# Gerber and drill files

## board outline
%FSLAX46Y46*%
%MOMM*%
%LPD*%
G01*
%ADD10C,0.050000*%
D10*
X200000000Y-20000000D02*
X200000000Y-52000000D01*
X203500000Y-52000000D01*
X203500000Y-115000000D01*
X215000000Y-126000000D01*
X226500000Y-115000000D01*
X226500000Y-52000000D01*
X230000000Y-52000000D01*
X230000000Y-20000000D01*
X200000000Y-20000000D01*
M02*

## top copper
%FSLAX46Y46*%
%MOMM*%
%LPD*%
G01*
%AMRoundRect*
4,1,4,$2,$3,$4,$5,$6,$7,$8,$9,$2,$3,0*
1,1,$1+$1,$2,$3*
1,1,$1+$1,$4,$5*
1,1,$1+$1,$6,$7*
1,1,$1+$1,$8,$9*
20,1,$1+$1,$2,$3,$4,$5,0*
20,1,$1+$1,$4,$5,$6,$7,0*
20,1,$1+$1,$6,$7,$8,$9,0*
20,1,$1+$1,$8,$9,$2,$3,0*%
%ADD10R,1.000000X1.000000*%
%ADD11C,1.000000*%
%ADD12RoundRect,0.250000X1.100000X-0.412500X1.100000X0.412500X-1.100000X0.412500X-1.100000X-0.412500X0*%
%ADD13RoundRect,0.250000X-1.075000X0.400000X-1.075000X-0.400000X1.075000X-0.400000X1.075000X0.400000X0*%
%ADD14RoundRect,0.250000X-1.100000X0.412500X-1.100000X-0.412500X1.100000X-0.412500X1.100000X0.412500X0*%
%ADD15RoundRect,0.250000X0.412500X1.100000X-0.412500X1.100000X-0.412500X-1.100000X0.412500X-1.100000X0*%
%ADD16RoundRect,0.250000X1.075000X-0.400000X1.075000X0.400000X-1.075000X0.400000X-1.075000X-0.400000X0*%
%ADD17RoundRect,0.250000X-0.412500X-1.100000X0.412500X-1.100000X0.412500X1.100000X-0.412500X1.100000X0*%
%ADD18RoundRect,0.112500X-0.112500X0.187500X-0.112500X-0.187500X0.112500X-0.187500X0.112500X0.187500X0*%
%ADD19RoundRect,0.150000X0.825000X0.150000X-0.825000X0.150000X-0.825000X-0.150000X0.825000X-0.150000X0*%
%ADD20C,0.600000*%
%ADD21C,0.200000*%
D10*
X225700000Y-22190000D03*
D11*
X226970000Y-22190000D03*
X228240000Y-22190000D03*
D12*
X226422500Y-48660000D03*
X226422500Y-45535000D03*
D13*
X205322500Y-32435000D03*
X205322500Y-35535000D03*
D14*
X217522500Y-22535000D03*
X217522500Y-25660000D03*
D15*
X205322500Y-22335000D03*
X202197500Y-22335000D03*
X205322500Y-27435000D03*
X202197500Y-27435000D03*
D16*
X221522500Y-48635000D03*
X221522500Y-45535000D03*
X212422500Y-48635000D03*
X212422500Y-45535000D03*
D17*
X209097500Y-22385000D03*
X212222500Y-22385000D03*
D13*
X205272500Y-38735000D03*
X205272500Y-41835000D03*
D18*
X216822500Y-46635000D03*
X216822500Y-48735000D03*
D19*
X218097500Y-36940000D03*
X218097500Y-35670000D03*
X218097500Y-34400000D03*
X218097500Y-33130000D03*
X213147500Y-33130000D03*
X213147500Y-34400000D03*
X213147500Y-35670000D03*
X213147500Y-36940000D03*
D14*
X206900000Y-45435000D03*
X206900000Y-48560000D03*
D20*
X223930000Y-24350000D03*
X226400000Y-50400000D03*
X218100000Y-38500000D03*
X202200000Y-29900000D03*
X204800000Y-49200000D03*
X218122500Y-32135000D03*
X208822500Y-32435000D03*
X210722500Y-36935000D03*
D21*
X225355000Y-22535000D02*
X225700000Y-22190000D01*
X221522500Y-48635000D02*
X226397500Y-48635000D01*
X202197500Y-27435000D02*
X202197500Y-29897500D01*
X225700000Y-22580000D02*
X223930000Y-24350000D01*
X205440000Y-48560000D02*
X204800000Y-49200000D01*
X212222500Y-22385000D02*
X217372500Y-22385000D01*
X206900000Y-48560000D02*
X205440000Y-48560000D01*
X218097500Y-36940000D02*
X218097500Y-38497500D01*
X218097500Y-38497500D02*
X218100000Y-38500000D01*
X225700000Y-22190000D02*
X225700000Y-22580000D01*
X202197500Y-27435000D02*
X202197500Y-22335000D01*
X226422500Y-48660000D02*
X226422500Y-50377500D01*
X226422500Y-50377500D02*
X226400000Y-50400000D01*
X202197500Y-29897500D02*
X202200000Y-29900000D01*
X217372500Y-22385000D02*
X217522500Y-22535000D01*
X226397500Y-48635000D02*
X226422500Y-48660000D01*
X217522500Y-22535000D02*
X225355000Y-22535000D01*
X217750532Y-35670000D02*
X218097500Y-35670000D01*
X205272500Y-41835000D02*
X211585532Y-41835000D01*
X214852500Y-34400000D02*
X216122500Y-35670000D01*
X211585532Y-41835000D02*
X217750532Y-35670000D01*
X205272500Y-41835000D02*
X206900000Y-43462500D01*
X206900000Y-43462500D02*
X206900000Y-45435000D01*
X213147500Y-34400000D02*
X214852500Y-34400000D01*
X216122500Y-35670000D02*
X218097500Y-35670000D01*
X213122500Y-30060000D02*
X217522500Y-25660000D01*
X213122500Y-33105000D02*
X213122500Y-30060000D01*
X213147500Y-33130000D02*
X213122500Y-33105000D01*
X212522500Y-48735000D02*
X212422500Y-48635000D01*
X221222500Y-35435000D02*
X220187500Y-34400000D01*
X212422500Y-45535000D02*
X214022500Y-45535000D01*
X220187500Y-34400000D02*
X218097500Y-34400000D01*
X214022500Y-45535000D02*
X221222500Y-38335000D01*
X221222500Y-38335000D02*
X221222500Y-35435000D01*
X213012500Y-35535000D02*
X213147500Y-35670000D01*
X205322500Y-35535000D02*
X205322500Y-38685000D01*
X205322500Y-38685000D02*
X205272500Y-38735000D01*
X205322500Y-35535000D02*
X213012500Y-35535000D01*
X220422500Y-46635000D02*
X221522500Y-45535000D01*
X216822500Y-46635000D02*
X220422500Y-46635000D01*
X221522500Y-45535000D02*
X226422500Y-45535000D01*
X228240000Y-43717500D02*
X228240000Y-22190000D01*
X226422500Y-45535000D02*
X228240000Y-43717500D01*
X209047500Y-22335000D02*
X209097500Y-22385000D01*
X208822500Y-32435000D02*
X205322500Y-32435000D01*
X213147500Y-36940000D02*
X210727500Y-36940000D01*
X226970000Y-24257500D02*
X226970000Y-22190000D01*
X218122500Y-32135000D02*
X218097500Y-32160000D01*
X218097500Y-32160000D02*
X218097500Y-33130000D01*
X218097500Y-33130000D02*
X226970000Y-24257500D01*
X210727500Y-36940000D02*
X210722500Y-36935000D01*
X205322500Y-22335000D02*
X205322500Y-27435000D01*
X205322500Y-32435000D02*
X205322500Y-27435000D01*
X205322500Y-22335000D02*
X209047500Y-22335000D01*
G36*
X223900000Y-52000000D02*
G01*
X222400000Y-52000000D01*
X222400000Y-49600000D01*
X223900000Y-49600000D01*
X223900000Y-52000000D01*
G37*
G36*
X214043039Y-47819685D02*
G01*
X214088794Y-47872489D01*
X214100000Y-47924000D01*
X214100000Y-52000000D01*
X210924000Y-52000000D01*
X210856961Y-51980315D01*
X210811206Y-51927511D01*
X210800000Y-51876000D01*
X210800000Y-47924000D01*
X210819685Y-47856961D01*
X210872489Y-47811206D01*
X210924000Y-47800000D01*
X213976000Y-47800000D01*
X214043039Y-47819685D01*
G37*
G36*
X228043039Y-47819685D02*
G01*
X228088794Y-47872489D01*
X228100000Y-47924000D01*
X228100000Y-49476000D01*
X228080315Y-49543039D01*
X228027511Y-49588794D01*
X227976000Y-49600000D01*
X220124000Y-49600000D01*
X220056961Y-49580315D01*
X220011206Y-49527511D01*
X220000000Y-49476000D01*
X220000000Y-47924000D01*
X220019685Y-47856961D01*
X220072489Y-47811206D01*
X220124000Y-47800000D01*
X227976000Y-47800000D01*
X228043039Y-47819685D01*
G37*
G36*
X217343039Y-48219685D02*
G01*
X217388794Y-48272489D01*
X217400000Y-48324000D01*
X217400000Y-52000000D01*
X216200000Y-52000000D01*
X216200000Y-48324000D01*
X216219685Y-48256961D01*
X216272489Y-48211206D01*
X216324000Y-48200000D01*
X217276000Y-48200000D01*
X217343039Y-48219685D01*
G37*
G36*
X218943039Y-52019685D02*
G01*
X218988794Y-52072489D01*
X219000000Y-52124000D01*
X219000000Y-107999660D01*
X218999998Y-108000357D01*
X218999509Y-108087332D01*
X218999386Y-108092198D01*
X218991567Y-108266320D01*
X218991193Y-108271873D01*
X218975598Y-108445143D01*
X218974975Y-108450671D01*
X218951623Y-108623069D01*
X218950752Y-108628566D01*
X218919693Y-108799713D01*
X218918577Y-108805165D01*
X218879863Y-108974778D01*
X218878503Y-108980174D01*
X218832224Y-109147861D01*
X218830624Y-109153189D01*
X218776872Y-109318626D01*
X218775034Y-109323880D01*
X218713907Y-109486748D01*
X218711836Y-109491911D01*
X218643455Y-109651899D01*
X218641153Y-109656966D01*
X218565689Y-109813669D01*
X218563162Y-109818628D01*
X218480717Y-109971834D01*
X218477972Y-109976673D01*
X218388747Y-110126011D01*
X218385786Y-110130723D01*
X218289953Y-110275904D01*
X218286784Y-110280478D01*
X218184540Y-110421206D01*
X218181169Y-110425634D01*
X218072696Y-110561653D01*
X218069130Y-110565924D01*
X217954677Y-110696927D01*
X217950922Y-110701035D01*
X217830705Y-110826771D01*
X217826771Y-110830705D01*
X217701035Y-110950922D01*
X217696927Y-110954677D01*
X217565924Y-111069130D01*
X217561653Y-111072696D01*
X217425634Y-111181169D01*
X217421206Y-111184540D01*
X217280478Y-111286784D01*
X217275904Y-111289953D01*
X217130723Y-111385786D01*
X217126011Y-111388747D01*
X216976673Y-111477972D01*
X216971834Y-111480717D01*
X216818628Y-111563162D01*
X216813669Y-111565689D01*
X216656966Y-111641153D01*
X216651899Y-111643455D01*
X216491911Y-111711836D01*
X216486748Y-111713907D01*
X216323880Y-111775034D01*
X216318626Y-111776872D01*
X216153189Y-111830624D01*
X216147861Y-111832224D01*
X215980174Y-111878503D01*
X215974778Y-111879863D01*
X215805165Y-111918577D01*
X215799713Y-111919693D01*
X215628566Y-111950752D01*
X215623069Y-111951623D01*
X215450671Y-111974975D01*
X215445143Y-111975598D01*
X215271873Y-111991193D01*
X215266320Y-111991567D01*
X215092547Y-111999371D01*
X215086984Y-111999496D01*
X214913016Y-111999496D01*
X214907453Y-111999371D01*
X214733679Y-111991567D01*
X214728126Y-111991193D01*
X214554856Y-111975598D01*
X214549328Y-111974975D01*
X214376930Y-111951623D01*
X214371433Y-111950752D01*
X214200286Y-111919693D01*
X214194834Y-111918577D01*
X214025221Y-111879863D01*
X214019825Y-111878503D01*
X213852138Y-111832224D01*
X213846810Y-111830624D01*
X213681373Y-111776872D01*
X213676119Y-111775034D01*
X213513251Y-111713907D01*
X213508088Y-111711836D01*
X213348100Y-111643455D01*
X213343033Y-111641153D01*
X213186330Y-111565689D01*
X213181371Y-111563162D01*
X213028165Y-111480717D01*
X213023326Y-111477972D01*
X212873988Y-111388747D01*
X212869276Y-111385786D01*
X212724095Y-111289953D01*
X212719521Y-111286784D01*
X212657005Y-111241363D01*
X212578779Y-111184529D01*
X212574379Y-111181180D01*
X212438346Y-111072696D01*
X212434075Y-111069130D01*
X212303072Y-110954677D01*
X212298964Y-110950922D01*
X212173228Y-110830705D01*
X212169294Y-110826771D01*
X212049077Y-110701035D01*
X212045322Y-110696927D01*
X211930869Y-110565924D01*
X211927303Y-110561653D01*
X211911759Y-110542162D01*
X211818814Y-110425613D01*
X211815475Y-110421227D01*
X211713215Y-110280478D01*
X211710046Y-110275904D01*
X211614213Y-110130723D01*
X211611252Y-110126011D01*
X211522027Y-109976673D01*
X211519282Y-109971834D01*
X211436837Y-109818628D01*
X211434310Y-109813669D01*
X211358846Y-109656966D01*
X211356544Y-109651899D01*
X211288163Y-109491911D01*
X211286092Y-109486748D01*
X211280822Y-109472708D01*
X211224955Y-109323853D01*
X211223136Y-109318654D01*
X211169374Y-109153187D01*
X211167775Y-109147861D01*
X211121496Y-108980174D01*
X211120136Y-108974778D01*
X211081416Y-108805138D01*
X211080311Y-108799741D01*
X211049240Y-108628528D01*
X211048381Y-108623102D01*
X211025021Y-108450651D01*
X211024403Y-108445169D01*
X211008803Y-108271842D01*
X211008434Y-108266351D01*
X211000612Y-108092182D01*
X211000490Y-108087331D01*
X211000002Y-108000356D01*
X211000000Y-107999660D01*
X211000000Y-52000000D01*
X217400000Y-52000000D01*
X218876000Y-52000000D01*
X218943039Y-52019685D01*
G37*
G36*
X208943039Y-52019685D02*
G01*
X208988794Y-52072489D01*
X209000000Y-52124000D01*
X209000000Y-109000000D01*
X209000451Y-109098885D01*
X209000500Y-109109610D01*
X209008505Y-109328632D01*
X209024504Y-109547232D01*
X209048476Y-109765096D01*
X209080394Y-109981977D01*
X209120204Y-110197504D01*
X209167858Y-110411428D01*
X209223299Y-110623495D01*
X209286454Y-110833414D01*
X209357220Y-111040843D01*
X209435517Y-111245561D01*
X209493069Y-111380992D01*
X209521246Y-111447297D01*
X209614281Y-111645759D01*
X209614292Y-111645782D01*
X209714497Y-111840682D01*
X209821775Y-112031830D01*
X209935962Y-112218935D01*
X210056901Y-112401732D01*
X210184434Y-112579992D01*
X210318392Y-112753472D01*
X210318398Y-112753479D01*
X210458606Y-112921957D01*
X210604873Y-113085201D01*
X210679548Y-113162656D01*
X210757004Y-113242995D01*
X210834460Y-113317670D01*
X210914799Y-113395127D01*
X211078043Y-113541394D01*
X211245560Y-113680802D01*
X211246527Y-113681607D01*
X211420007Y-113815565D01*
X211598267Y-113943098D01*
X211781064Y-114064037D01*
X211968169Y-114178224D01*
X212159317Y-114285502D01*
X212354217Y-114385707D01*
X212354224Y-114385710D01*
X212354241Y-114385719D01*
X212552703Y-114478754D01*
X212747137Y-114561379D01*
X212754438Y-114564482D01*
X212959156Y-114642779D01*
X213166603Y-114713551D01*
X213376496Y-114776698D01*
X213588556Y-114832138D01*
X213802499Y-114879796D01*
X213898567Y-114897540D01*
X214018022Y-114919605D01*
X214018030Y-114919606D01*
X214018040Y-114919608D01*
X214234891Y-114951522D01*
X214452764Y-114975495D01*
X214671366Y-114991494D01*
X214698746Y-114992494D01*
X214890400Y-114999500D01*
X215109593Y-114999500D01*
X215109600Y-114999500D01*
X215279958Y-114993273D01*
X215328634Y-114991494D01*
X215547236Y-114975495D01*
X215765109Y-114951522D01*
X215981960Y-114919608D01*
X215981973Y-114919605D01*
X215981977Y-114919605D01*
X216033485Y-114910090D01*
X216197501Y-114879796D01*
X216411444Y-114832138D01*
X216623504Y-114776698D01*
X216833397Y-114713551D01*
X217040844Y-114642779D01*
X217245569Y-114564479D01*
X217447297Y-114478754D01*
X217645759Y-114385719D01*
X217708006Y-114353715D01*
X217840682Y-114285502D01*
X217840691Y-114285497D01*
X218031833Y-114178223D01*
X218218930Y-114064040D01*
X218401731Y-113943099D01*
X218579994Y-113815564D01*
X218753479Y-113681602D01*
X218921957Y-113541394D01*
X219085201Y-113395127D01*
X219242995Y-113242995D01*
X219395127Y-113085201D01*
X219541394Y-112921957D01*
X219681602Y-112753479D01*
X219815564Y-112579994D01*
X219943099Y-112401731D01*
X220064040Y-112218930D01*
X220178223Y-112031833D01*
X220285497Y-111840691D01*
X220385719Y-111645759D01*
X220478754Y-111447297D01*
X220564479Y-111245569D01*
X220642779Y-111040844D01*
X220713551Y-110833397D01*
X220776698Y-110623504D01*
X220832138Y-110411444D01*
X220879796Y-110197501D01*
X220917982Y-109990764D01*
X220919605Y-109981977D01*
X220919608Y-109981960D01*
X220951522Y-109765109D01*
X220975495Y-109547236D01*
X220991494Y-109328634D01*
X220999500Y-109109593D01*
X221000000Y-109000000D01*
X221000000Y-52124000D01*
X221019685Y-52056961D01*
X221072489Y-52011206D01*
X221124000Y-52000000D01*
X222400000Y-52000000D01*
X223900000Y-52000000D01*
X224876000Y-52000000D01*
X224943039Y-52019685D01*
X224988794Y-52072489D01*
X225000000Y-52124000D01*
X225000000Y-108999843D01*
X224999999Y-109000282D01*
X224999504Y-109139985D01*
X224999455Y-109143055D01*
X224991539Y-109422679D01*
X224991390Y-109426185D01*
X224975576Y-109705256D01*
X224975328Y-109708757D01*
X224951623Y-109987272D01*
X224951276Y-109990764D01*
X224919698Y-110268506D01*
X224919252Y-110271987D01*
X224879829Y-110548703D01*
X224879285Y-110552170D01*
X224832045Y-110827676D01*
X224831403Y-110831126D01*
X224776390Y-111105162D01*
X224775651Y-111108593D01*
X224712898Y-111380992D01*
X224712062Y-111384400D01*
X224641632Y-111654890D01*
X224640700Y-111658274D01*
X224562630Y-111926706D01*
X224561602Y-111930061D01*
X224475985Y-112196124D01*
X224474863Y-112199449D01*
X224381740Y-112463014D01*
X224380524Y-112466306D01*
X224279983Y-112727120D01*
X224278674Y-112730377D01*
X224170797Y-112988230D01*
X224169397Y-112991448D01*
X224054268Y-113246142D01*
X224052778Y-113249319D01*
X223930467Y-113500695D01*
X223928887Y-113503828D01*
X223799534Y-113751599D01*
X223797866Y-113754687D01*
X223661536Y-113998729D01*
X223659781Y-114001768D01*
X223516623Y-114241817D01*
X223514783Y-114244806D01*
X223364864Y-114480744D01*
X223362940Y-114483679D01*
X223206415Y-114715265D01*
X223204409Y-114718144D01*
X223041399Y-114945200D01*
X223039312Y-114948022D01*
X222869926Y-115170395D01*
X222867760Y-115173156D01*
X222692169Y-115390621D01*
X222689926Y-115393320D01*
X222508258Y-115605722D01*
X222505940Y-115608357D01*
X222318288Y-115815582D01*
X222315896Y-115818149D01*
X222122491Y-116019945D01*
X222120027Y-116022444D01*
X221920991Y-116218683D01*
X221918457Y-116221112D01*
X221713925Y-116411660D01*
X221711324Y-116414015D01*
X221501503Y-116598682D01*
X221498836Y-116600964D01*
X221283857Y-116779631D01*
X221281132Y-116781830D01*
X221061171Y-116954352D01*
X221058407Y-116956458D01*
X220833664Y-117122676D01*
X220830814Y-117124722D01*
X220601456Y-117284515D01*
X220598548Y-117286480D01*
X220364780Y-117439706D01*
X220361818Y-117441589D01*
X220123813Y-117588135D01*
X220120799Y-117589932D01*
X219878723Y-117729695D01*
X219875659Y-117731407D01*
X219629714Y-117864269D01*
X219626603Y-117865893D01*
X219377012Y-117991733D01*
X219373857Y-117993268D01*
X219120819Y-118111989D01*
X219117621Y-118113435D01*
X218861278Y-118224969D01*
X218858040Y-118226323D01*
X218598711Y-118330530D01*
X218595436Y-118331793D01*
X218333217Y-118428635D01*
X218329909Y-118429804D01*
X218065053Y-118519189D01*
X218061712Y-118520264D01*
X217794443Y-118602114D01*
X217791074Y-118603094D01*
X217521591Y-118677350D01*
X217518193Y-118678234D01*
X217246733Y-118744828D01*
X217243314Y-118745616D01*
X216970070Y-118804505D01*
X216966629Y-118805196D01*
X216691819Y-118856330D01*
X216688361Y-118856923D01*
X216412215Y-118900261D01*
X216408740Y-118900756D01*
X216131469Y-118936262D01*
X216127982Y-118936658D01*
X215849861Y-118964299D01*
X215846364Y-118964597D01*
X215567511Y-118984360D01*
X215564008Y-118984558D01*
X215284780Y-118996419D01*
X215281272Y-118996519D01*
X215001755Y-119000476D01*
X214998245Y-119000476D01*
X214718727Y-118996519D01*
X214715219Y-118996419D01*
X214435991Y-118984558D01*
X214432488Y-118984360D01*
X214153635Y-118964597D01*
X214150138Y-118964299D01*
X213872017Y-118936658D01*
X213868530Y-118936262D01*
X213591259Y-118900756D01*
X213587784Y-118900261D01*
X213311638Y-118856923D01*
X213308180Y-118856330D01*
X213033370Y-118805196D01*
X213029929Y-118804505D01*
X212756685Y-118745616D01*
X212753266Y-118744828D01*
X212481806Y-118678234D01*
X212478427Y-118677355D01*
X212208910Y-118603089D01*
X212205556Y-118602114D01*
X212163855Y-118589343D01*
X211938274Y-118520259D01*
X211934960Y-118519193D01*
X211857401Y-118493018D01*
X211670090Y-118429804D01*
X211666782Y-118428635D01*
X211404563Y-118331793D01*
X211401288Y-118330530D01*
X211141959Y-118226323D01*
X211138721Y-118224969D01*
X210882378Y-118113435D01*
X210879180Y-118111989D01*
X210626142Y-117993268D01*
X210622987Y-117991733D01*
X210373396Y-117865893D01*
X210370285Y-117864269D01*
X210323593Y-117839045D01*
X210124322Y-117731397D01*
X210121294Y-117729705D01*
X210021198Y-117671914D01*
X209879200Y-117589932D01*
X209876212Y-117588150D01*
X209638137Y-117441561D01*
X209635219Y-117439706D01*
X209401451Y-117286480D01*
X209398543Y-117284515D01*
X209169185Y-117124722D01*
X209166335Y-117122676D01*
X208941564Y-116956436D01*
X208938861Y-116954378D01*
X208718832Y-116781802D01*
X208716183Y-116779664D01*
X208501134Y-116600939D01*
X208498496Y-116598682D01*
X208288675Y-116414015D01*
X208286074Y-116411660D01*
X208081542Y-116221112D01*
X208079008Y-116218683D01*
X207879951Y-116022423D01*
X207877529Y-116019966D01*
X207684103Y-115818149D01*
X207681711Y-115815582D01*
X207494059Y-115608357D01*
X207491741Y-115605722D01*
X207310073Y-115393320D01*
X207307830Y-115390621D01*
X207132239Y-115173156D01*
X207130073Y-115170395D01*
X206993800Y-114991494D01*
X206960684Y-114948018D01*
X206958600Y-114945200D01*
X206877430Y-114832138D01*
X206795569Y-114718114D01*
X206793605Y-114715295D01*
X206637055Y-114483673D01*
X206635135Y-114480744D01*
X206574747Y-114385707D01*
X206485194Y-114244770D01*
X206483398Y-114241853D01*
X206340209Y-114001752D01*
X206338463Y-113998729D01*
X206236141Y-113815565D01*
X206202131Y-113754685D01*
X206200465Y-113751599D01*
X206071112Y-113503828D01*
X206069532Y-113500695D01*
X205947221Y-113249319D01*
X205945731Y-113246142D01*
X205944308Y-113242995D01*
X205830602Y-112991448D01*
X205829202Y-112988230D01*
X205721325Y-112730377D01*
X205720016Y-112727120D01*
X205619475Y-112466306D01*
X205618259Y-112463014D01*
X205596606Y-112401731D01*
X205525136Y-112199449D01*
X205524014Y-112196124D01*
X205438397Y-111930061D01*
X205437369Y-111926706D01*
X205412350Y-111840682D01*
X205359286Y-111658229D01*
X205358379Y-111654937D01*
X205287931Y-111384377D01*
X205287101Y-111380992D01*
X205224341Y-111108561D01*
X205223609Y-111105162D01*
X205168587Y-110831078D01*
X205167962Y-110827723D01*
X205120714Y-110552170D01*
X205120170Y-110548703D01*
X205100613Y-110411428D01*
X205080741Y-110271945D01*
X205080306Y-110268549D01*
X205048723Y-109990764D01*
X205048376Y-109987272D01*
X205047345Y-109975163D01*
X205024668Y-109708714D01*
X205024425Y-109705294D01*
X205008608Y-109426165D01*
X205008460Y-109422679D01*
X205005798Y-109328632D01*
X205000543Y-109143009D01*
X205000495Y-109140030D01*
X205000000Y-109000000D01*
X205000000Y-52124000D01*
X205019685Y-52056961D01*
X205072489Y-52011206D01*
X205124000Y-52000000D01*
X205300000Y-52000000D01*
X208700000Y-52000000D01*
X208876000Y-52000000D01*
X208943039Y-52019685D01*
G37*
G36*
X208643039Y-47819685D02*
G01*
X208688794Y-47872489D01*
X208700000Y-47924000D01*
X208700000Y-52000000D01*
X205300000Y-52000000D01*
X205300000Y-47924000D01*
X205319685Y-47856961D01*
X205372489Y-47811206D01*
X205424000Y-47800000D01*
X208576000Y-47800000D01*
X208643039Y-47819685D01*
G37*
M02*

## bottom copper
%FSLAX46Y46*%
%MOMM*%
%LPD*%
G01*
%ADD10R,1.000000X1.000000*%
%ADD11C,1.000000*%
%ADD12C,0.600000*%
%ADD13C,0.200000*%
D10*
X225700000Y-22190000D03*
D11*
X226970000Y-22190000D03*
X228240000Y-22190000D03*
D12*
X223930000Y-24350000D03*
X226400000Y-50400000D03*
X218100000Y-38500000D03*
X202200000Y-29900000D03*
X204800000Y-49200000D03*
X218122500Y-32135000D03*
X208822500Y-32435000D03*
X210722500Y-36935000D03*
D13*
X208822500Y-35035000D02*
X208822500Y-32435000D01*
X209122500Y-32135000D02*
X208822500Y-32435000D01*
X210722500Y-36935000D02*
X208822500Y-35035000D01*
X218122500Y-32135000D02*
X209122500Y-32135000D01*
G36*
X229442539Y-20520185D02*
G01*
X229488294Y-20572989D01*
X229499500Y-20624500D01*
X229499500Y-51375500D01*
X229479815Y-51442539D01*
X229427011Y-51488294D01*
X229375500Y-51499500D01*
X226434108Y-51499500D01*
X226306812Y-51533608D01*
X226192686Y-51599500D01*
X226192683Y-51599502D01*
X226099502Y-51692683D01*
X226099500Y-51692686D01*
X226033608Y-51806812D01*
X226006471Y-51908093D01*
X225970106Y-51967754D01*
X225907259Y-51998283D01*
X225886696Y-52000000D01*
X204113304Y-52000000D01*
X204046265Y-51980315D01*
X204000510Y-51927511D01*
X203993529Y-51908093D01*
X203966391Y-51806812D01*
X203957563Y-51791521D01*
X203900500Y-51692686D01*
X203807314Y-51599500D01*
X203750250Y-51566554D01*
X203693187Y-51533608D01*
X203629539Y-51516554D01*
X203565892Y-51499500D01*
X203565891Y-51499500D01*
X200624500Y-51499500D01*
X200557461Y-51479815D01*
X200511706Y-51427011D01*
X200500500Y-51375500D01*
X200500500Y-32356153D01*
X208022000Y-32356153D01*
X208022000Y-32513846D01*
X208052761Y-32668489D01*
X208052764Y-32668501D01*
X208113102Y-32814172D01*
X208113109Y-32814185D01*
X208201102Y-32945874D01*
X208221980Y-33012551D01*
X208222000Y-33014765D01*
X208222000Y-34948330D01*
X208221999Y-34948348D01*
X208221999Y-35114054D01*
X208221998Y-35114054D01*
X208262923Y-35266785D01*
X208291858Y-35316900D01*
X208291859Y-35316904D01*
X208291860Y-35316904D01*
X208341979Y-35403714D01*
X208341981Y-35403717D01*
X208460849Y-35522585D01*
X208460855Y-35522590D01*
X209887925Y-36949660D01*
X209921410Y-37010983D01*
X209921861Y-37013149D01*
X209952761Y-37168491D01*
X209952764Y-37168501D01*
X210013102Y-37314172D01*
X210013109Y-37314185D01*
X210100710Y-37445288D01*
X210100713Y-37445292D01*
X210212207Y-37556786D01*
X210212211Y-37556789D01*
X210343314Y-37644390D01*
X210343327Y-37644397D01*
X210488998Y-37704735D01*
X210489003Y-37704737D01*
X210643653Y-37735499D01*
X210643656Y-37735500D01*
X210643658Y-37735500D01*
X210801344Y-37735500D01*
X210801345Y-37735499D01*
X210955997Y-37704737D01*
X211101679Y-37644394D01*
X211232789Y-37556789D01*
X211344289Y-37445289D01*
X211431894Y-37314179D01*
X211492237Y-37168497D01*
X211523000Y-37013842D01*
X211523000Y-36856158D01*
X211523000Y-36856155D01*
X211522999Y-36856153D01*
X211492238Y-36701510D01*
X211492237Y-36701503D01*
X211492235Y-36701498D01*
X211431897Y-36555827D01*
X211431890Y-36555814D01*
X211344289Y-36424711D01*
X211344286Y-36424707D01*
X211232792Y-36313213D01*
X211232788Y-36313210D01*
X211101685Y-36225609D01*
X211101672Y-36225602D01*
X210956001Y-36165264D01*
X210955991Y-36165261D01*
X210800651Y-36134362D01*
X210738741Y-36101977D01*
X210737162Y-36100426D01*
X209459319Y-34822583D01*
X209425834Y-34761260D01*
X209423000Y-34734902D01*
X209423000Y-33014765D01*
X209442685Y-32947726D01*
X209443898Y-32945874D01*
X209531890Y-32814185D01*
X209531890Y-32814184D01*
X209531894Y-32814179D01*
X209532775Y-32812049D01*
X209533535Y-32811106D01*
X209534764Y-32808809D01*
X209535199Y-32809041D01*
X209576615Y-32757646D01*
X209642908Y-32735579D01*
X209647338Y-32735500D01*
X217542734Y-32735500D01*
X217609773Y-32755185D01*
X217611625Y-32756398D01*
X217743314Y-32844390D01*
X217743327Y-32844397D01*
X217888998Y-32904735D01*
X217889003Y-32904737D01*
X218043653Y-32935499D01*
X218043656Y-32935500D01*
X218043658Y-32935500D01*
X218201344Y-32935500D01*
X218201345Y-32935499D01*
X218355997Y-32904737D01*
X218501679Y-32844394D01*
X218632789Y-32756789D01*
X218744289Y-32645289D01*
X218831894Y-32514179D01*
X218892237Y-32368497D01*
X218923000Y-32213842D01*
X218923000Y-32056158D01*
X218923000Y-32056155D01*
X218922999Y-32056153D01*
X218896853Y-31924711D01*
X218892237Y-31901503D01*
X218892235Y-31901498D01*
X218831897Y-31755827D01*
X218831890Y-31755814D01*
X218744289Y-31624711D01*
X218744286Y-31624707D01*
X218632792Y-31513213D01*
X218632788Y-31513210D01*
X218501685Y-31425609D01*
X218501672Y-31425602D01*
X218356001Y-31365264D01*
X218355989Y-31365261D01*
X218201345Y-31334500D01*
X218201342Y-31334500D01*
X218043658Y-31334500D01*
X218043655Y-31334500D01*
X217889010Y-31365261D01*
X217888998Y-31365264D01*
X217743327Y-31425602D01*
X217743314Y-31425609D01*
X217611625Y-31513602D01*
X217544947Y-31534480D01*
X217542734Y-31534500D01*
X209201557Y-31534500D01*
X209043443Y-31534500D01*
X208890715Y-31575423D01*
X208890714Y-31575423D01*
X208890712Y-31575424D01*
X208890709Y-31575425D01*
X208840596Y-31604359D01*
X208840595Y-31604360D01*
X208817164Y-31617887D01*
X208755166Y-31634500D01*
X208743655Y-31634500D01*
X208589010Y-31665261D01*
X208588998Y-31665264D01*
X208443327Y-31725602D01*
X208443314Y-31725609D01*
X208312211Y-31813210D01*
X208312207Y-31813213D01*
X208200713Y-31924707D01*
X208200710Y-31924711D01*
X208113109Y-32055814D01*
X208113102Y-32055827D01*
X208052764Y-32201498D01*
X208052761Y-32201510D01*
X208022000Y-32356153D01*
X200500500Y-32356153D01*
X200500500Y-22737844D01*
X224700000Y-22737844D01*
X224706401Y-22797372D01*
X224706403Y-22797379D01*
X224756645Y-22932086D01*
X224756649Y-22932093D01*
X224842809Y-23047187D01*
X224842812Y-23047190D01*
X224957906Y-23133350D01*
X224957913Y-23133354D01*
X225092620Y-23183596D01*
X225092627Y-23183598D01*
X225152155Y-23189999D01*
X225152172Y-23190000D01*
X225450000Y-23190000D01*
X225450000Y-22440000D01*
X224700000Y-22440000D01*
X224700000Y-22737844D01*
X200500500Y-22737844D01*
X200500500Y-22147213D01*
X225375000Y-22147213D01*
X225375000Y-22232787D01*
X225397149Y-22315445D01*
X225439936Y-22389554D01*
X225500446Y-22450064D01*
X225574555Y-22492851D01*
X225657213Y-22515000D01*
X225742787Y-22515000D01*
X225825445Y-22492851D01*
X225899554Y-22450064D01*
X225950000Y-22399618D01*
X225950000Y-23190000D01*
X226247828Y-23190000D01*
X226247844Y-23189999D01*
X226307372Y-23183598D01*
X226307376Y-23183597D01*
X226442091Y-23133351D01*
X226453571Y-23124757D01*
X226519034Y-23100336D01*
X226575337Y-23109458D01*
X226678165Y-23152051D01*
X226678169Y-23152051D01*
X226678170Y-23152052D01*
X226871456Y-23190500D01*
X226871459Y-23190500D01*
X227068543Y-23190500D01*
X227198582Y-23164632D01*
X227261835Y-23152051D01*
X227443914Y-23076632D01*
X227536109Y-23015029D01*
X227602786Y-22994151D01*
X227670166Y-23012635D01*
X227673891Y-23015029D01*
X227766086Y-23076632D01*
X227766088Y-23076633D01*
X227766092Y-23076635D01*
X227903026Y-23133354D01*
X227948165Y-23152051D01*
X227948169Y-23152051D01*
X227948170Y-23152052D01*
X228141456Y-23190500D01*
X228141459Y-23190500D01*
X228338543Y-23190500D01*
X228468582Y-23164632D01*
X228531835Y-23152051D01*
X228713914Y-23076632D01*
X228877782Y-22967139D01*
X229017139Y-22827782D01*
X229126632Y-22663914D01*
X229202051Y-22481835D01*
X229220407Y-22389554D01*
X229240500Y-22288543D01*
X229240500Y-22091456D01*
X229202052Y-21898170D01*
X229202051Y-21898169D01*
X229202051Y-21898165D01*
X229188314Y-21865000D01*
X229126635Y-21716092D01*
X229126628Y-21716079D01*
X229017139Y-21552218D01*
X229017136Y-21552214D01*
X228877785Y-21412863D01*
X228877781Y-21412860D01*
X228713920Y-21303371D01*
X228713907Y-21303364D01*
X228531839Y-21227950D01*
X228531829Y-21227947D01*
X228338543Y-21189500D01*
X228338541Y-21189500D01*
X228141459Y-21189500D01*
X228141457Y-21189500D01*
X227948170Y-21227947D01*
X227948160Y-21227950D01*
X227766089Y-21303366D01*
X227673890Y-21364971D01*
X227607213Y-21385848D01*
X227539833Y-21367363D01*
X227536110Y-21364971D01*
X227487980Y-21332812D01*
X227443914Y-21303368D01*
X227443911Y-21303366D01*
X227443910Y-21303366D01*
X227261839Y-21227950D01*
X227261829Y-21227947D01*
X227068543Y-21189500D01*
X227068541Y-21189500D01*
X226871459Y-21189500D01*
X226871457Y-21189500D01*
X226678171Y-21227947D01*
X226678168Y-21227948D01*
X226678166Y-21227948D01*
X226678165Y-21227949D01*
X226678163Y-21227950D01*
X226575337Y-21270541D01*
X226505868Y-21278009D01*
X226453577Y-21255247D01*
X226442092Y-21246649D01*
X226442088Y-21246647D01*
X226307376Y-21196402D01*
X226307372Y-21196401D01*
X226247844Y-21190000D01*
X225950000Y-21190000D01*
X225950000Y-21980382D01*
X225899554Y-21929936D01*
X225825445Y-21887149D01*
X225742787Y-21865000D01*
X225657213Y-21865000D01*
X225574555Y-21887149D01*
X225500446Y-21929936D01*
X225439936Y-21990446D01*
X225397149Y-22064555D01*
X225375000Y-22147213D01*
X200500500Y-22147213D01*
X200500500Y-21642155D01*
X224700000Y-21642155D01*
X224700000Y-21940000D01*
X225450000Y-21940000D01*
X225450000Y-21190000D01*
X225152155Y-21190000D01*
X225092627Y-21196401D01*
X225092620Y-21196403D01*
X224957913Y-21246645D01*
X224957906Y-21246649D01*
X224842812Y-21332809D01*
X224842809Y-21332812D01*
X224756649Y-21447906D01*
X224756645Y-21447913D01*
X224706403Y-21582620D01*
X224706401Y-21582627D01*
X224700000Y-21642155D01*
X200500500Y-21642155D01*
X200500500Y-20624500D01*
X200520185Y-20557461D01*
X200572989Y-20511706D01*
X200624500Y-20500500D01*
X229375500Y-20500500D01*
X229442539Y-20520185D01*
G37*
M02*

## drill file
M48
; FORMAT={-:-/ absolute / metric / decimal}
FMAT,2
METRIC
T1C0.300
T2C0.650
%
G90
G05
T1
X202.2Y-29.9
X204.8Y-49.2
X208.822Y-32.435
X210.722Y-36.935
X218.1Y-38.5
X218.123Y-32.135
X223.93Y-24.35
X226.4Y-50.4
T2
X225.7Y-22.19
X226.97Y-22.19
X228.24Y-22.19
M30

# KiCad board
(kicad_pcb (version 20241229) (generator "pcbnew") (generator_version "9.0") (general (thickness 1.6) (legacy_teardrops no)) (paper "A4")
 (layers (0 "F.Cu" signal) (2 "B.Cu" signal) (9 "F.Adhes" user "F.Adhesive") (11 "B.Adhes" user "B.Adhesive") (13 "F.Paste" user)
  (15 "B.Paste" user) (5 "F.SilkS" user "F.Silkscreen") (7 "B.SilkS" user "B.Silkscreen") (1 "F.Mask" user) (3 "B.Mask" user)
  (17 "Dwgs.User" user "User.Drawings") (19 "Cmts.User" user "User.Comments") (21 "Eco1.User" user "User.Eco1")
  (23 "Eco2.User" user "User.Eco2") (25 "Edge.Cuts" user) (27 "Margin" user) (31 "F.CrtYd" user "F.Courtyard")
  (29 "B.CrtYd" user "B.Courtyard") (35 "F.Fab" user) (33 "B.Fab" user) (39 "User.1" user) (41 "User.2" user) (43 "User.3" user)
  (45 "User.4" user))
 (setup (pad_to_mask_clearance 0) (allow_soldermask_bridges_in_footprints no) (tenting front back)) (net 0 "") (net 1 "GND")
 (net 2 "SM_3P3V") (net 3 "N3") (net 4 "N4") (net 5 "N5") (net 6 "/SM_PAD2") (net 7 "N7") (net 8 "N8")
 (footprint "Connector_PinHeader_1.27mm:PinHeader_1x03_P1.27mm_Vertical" (layer "F.Cu") (at 225.7 22.19 90)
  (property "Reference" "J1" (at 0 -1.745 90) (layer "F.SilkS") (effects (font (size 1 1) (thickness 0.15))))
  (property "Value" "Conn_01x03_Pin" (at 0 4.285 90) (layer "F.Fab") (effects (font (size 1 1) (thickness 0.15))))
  (pad "1" thru_hole rect (at 0 0 90) (size 1 1) (drill 0.65) (layers "*.Cu" "*.Mask") (remove_unused_layers no) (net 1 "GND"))
  (pad "2" thru_hole circle (at 0 1.27 90) (size 1 1) (drill 0.65) (layers "*.Cu" "*.Mask") (remove_unused_layers no) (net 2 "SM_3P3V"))
  (pad "3" thru_hole circle (at 0 2.54 90) (size 1 1) (drill 0.65) (layers "*.Cu" "*.Mask") (remove_unused_layers no) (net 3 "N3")))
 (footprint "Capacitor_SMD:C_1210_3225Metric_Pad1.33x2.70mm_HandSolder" (layer "F.Cu") (at 226.4225 47.0975 90)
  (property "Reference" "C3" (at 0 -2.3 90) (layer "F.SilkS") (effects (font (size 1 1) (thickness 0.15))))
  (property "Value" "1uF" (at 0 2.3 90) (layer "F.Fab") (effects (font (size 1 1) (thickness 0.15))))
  (pad "1" smd roundrect (at -1.5625 0 90) (size 1.325 2.7) (layers "F.Cu" "F.Mask" "F.Paste") (roundrect_rratio 0.188679) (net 1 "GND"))
  (pad "2" smd roundrect (at 1.5625 0 90) (size 1.325 2.7) (layers "F.Cu" "F.Mask" "F.Paste") (roundrect_rratio 0.188679) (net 3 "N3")))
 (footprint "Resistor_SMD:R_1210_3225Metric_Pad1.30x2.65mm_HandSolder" (layer "F.Cu") (at 205.3225 33.985 -90)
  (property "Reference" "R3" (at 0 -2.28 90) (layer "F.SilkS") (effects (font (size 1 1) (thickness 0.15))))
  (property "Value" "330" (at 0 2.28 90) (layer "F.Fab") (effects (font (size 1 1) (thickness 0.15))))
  (pad "1" smd roundrect (at -1.55 0 270) (size 1.3 2.65) (layers "F.Cu" "F.Mask" "F.Paste") (roundrect_rratio 0.192308) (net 2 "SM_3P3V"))
  (pad "2" smd roundrect (at 1.55 0 270) (size 1.3 2.65) (layers "F.Cu" "F.Mask" "F.Paste") (roundrect_rratio 0.192308) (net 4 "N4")))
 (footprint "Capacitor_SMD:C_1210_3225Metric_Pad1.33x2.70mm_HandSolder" (layer "F.Cu") (at 217.5225 24.0975 -90)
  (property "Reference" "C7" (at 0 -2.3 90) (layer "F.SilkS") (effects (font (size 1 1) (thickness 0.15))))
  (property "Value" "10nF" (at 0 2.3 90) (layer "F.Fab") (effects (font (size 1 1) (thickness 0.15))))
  (pad "1" smd roundrect (at -1.5625 0 270) (size 1.325 2.7) (layers "F.Cu" "F.Mask" "F.Paste") (roundrect_rratio 0.188679) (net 1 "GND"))
  (pad "2" smd roundrect (at 1.5625 0 270) (size 1.325 2.7) (layers "F.Cu" "F.Mask" "F.Paste") (roundrect_rratio 0.188679) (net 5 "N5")))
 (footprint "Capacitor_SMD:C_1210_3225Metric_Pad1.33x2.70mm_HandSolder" (layer "F.Cu") (at 203.76 22.335 180)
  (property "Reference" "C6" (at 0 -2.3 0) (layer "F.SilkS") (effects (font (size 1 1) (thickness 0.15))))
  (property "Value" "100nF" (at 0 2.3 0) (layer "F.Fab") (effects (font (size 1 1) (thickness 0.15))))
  (pad "1" smd roundrect (at -1.5625 0 180) (size 1.325 2.7) (layers "F.Cu" "F.Mask" "F.Paste") (roundrect_rratio 0.188679)
   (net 2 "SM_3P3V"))
  (pad "2" smd roundrect (at 1.5625 0 180) (size 1.325 2.7) (layers "F.Cu" "F.Mask" "F.Paste") (roundrect_rratio 0.188679) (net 1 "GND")))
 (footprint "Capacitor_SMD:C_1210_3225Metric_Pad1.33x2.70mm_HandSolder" (layer "F.Cu") (at 203.76 27.435 180)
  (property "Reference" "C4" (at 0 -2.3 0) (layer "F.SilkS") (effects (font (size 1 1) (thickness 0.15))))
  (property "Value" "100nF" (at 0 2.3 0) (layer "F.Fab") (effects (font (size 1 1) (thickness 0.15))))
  (pad "1" smd roundrect (at -1.5625 0 180) (size 1.325 2.7) (layers "F.Cu" "F.Mask" "F.Paste") (roundrect_rratio 0.188679)
   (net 2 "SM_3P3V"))
  (pad "2" smd roundrect (at 1.5625 0 180) (size 1.325 2.7) (layers "F.Cu" "F.Mask" "F.Paste") (roundrect_rratio 0.188679) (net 1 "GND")))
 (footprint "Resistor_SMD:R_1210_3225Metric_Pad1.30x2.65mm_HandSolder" (layer "F.Cu") (at 221.5225 47.085 90)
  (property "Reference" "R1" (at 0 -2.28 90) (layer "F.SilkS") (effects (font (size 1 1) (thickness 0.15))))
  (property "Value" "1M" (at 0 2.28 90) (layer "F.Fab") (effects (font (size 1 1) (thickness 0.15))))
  (pad "1" smd roundrect (at -1.55 0 90) (size 1.3 2.65) (layers "F.Cu" "F.Mask" "F.Paste") (roundrect_rratio 0.192308) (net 1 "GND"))
  (pad "2" smd roundrect (at 1.55 0 90) (size 1.3 2.65) (layers "F.Cu" "F.Mask" "F.Paste") (roundrect_rratio 0.192308) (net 3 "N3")))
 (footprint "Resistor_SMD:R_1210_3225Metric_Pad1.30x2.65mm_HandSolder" (layer "F.Cu") (at 212.4225 47.085 90)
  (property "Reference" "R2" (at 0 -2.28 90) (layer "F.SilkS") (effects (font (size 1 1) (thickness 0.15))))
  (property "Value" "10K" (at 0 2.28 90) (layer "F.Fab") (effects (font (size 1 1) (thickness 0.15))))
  (pad "1" smd roundrect (at -1.55 0 90) (size 1.3 2.65) (layers "F.Cu" "F.Mask" "F.Paste") (roundrect_rratio 0.192308) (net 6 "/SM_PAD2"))
  (pad "2" smd roundrect (at 1.55 0 90) (size 1.3 2.65) (layers "F.Cu" "F.Mask" "F.Paste") (roundrect_rratio 0.192308) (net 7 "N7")))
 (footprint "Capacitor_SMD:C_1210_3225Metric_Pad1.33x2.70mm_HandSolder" (layer "F.Cu") (at 210.66 22.385)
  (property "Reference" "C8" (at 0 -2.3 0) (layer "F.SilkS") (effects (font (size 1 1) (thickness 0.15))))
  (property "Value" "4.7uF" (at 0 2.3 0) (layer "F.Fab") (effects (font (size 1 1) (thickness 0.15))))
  (pad "1" smd roundrect (at -1.5625 0) (size 1.325 2.7) (layers "F.Cu" "F.Mask" "F.Paste") (roundrect_rratio 0.188679) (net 2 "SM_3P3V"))
  (pad "2" smd roundrect (at 1.5625 0) (size 1.325 2.7) (layers "F.Cu" "F.Mask" "F.Paste") (roundrect_rratio 0.188679) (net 1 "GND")))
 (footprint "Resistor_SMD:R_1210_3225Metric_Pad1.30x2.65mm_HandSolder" (layer "F.Cu") (at 205.2725 40.285 -90)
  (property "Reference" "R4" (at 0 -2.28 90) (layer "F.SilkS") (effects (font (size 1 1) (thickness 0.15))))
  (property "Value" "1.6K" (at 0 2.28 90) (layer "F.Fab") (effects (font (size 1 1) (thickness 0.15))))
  (pad "1" smd roundrect (at -1.55 0 270) (size 1.3 2.65) (layers "F.Cu" "F.Mask" "F.Paste") (roundrect_rratio 0.192308) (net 4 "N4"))
  (pad "2" smd roundrect (at 1.55 0 270) (size 1.3 2.65) (layers "F.Cu" "F.Mask" "F.Paste") (roundrect_rratio 0.192308) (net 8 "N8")))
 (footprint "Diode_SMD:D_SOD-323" (layer "F.Cu") (at 216.8225 47.685 -90)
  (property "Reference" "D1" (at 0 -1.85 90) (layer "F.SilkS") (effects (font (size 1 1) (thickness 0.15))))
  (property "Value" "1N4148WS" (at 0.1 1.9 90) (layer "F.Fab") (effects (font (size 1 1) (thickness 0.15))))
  (pad "1" smd roundrect (at -1.05 0 270) (size 0.6 0.45) (layers "F.Cu" "F.Mask" "F.Paste") (roundrect_rratio 0.25) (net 3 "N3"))
  (pad "2" smd roundrect (at 1.05 0 270) (size 0.6 0.45) (layers "F.Cu" "F.Mask" "F.Paste") (roundrect_rratio 0.25) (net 6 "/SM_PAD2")))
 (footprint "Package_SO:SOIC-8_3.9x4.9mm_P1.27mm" (layer "F.Cu") (at 215.6225 35.035 180)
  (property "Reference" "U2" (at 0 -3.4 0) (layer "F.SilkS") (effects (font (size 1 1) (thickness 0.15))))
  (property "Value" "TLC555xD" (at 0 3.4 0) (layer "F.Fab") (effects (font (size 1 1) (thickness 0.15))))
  (pad "1" smd roundrect (at -2.475 -1.905 180) (size 1.95 0.6) (layers "F.Cu" "F.Mask" "F.Paste") (roundrect_rratio 0.25) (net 1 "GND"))
  (pad "2" smd roundrect (at -2.475 -0.635 180) (size 1.95 0.6) (layers "F.Cu" "F.Mask" "F.Paste") (roundrect_rratio 0.25) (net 8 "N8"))
  (pad "3" smd roundrect (at -2.475 0.635 180) (size 1.95 0.6) (layers "F.Cu" "F.Mask" "F.Paste") (roundrect_rratio 0.25) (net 7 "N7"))
  (pad "4" smd roundrect (at -2.475 1.905 180) (size 1.95 0.6) (layers "F.Cu" "F.Mask" "F.Paste") (roundrect_rratio 0.25) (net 2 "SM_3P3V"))
  (pad "5" smd roundrect (at 2.475 1.905 180) (size 1.95 0.6) (layers "F.Cu" "F.Mask" "F.Paste") (roundrect_rratio 0.25) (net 5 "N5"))
  (pad "6" smd roundrect (at 2.475 0.635 180) (size 1.95 0.6) (layers "F.Cu" "F.Mask" "F.Paste") (roundrect_rratio 0.25) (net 8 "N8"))
  (pad "7" smd roundrect (at 2.475 -0.635 180) (size 1.95 0.6) (layers "F.Cu" "F.Mask" "F.Paste") (roundrect_rratio 0.25) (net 4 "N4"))
  (pad "8" smd roundrect (at 2.475 -1.905 180) (size 1.95 0.6) (layers "F.Cu" "F.Mask" "F.Paste") (roundrect_rratio 0.25) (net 2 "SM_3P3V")))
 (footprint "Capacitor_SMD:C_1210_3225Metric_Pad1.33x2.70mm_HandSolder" (layer "F.Cu") (at 206.9 46.9975 -90)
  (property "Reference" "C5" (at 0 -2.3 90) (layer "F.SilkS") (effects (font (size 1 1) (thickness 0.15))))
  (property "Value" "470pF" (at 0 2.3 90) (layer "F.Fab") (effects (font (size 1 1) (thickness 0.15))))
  (pad "1" smd roundrect (at -1.5625 0 270) (size 1.325 2.7) (layers "F.Cu" "F.Mask" "F.Paste") (roundrect_rratio 0.188679) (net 8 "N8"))
  (pad "2" smd roundrect (at 1.5625 0 270) (size 1.325 2.7) (layers "F.Cu" "F.Mask" "F.Paste") (roundrect_rratio 0.188679) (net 1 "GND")))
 (gr_poly
  (pts (xy 200 20) (xy 200 52) (xy 203.5 52) (xy 203.5 115) (xy 215 126) (xy 226.5 115) (xy 226.5 52) (xy 230 52) (xy 230 20))
  (stroke (width 0.05) (type solid)) (fill no) (layer "Edge.Cuts"))
 (segment (start 225.355 22.535) (end 225.7 22.19) (width 0.2) (layer "F.Cu") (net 1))
 (segment (start 221.5225 48.635) (end 226.3975 48.635) (width 0.2) (layer "F.Cu") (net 1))
 (segment (start 202.1975 27.435) (end 202.1975 29.8975) (width 0.2) (layer "F.Cu") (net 1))
 (segment (start 225.7 22.58) (end 223.93 24.35) (width 0.2) (layer "F.Cu") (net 1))
 (segment (start 205.44 48.56) (end 204.8 49.2) (width 0.2) (layer "F.Cu") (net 1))
 (segment (start 212.2225 22.385) (end 217.3725 22.385) (width 0.2) (layer "F.Cu") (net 1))
 (segment (start 206.9 48.56) (end 205.44 48.56) (width 0.2) (layer "F.Cu") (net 1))
 (segment (start 218.0975 36.94) (end 218.0975 38.4975) (width 0.2) (layer "F.Cu") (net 1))
 (segment (start 218.0975 38.4975) (end 218.1 38.5) (width 0.2) (layer "F.Cu") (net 1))
 (segment (start 225.7 22.19) (end 225.7 22.58) (width 0.2) (layer "F.Cu") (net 1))
 (segment (start 202.1975 27.435) (end 202.1975 22.335) (width 0.2) (layer "F.Cu") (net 1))
 (segment (start 226.4225 48.66) (end 226.4225 50.3775) (width 0.2) (layer "F.Cu") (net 1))
 (segment (start 226.4225 50.3775) (end 226.4 50.4) (width 0.2) (layer "F.Cu") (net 1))
 (segment (start 202.1975 29.8975) (end 202.2 29.9) (width 0.2) (layer "F.Cu") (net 1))
 (segment (start 217.3725 22.385) (end 217.5225 22.535) (width 0.2) (layer "F.Cu") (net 1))
 (segment (start 226.3975 48.635) (end 226.4225 48.66) (width 0.2) (layer "F.Cu") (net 1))
 (segment (start 217.5225 22.535) (end 225.355 22.535) (width 0.2) (layer "F.Cu") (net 1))
 (via (at 223.93 24.35) (size 0.6) (drill 0.3) (layers "F.Cu" "B.Cu") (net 1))
 (via (at 226.4 50.4) (size 0.6) (drill 0.3) (layers "F.Cu" "B.Cu") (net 1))
 (via (at 218.1 38.5) (size 0.6) (drill 0.3) (layers "F.Cu" "B.Cu") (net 1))
 (via (at 202.2 29.9) (size 0.6) (drill 0.3) (layers "F.Cu" "B.Cu") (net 1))
 (via (at 204.8 49.2) (size 0.6) (drill 0.3) (layers "F.Cu" "B.Cu") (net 1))
 (segment (start 217.750532 35.67) (end 218.0975 35.67) (width 0.2) (layer "F.Cu") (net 8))
 (segment (start 205.2725 41.835) (end 211.585532 41.835) (width 0.2) (layer "F.Cu") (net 8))
 (segment (start 214.8525 34.4) (end 216.1225 35.67) (width 0.2) (layer "F.Cu") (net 8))
 (segment (start 211.585532 41.835) (end 217.750532 35.67) (width 0.2) (layer "F.Cu") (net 8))
 (segment (start 205.2725 41.835) (end 206.9 43.4625) (width 0.2) (layer "F.Cu") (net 8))
 (segment (start 206.9 43.4625) (end 206.9 45.435) (width 0.2) (layer "F.Cu") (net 8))
 (segment (start 213.1475 34.4) (end 214.8525 34.4) (width 0.2) (layer "F.Cu") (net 8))
 (segment (start 216.1225 35.67) (end 218.0975 35.67) (width 0.2) (layer "F.Cu") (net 8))
 (segment (start 213.1225 30.06) (end 217.5225 25.66) (width 0.2) (layer "F.Cu") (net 5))
 (segment (start 213.1225 33.105) (end 213.1225 30.06) (width 0.2) (layer "F.Cu") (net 5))
 (segment (start 213.1475 33.13) (end 213.1225 33.105) (width 0.2) (layer "F.Cu") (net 5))
 (segment (start 212.5225 48.735) (end 212.4225 48.635) (width 0.2) (layer "F.Cu") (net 6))
 (segment (start 221.2225 35.435) (end 220.1875 34.4) (width 0.2) (layer "F.Cu") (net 7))
 (segment (start 212.4225 45.535) (end 214.0225 45.535) (width 0.2) (layer "F.Cu") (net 7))
 (segment (start 220.1875 34.4) (end 218.0975 34.4) (width 0.2) (layer "F.Cu") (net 7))
 (segment (start 214.0225 45.535) (end 221.2225 38.335) (width 0.2) (layer "F.Cu") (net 7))
 (segment (start 221.2225 38.335) (end 221.2225 35.435) (width 0.2) (layer "F.Cu") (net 7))
 (segment (start 213.0125 35.535) (end 213.1475 35.67) (width 0.2) (layer "F.Cu") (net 4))
 (segment (start 205.3225 35.535) (end 205.3225 38.685) (width 0.2) (layer "F.Cu") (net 4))
 (segment (start 205.3225 38.685) (end 205.2725 38.735) (width 0.2) (layer "F.Cu") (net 4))
 (segment (start 205.3225 35.535) (end 213.0125 35.535) (width 0.2) (layer "F.Cu") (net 4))
 (segment (start 220.4225 46.635) (end 221.5225 45.535) (width 0.2) (layer "F.Cu") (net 3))
 (segment (start 216.8225 46.635) (end 220.4225 46.635) (width 0.2) (layer "F.Cu") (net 3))
 (segment (start 221.5225 45.535) (end 226.4225 45.535) (width 0.2) (layer "F.Cu") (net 3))
 (segment (start 228.24 43.7175) (end 228.24 22.19) (width 0.2) (layer "F.Cu") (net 3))
 (segment (start 226.4225 45.535) (end 228.24 43.7175) (width 0.2) (layer "F.Cu") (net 3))
 (segment (start 209.0475 22.335) (end 209.0975 22.385) (width 0.2) (layer "F.Cu") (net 2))
 (segment (start 208.8225 32.435) (end 205.3225 32.435) (width 0.2) (layer "F.Cu") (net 2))
 (segment (start 213.1475 36.94) (end 210.7275 36.94) (width 0.2) (layer "F.Cu") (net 2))
 (segment (start 226.97 24.2575) (end 226.97 22.19) (width 0.2) (layer "F.Cu") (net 2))
 (segment (start 218.1225 32.135) (end 218.0975 32.16) (width 0.2) (layer "F.Cu") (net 2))
 (segment (start 218.0975 32.16) (end 218.0975 33.13) (width 0.2) (layer "F.Cu") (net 2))
 (segment (start 218.0975 33.13) (end 226.97 24.2575) (width 0.2) (layer "F.Cu") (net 2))
 (segment (start 210.7275 36.94) (end 210.7225 36.935) (width 0.2) (layer "F.Cu") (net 2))
 (segment (start 205.3225 22.335) (end 205.3225 27.435) (width 0.2) (layer "F.Cu") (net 2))
 (segment (start 205.3225 32.435) (end 205.3225 27.435) (width 0.2) (layer "F.Cu") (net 2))
 (segment (start 205.3225 22.335) (end 209.0475 22.335) (width 0.2) (layer "F.Cu") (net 2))
 (via (at 218.1225 32.135) (size 0.6) (drill 0.3) (layers "F.Cu" "B.Cu") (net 2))
 (via (at 208.8225 32.435) (size 0.6) (drill 0.3) (layers "F.Cu" "B.Cu") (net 2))
 (via (at 210.7225 36.935) (size 0.6) (drill 0.3) (layers "F.Cu" "B.Cu") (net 2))
 (segment (start 208.8225 35.035) (end 208.8225 32.435) (width 0.2) (layer "B.Cu") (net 2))
 (segment (start 209.1225 32.135) (end 208.8225 32.435) (width 0.2) (layer "B.Cu") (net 2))
 (segment (start 210.7225 36.935) (end 208.8225 35.035) (width 0.2) (layer "B.Cu") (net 2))
 (segment (start 218.1225 32.135) (end 209.1225 32.135) (width 0.2) (layer "B.Cu") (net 2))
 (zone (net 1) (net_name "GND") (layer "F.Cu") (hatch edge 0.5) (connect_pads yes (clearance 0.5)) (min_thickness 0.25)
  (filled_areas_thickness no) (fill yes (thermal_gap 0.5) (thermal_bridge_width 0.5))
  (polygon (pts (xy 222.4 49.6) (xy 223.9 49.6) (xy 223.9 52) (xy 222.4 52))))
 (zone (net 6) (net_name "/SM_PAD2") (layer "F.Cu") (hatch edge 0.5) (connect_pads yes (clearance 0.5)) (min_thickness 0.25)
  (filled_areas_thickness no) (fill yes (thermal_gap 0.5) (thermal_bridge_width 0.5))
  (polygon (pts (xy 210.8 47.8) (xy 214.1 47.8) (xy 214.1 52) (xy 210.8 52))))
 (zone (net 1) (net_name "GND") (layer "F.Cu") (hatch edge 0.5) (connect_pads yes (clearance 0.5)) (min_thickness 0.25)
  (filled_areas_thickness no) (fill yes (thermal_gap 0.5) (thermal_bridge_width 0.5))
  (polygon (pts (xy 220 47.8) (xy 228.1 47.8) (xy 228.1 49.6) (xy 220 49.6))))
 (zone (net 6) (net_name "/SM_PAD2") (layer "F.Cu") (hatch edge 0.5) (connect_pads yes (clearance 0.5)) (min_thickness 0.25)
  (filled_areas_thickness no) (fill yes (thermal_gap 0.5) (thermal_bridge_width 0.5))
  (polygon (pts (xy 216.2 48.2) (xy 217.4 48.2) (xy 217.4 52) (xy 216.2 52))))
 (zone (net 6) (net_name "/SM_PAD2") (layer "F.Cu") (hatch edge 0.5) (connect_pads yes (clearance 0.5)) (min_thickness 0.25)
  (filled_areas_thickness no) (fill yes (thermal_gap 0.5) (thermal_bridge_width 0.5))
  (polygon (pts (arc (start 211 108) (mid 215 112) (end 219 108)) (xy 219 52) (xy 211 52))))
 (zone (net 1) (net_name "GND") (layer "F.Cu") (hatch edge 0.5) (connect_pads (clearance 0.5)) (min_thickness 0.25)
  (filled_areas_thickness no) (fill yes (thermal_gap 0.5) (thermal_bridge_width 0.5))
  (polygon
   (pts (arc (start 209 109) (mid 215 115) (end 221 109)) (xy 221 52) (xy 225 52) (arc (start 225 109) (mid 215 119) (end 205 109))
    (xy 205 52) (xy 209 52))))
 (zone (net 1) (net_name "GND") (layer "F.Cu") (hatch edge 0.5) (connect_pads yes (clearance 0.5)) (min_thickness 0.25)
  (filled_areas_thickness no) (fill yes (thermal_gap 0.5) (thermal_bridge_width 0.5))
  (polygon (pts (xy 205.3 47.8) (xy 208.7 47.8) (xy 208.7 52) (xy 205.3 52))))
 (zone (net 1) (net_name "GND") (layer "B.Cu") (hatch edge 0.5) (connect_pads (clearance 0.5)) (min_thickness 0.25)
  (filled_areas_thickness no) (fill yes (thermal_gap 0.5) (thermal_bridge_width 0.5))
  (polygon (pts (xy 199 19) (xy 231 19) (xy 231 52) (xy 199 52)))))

